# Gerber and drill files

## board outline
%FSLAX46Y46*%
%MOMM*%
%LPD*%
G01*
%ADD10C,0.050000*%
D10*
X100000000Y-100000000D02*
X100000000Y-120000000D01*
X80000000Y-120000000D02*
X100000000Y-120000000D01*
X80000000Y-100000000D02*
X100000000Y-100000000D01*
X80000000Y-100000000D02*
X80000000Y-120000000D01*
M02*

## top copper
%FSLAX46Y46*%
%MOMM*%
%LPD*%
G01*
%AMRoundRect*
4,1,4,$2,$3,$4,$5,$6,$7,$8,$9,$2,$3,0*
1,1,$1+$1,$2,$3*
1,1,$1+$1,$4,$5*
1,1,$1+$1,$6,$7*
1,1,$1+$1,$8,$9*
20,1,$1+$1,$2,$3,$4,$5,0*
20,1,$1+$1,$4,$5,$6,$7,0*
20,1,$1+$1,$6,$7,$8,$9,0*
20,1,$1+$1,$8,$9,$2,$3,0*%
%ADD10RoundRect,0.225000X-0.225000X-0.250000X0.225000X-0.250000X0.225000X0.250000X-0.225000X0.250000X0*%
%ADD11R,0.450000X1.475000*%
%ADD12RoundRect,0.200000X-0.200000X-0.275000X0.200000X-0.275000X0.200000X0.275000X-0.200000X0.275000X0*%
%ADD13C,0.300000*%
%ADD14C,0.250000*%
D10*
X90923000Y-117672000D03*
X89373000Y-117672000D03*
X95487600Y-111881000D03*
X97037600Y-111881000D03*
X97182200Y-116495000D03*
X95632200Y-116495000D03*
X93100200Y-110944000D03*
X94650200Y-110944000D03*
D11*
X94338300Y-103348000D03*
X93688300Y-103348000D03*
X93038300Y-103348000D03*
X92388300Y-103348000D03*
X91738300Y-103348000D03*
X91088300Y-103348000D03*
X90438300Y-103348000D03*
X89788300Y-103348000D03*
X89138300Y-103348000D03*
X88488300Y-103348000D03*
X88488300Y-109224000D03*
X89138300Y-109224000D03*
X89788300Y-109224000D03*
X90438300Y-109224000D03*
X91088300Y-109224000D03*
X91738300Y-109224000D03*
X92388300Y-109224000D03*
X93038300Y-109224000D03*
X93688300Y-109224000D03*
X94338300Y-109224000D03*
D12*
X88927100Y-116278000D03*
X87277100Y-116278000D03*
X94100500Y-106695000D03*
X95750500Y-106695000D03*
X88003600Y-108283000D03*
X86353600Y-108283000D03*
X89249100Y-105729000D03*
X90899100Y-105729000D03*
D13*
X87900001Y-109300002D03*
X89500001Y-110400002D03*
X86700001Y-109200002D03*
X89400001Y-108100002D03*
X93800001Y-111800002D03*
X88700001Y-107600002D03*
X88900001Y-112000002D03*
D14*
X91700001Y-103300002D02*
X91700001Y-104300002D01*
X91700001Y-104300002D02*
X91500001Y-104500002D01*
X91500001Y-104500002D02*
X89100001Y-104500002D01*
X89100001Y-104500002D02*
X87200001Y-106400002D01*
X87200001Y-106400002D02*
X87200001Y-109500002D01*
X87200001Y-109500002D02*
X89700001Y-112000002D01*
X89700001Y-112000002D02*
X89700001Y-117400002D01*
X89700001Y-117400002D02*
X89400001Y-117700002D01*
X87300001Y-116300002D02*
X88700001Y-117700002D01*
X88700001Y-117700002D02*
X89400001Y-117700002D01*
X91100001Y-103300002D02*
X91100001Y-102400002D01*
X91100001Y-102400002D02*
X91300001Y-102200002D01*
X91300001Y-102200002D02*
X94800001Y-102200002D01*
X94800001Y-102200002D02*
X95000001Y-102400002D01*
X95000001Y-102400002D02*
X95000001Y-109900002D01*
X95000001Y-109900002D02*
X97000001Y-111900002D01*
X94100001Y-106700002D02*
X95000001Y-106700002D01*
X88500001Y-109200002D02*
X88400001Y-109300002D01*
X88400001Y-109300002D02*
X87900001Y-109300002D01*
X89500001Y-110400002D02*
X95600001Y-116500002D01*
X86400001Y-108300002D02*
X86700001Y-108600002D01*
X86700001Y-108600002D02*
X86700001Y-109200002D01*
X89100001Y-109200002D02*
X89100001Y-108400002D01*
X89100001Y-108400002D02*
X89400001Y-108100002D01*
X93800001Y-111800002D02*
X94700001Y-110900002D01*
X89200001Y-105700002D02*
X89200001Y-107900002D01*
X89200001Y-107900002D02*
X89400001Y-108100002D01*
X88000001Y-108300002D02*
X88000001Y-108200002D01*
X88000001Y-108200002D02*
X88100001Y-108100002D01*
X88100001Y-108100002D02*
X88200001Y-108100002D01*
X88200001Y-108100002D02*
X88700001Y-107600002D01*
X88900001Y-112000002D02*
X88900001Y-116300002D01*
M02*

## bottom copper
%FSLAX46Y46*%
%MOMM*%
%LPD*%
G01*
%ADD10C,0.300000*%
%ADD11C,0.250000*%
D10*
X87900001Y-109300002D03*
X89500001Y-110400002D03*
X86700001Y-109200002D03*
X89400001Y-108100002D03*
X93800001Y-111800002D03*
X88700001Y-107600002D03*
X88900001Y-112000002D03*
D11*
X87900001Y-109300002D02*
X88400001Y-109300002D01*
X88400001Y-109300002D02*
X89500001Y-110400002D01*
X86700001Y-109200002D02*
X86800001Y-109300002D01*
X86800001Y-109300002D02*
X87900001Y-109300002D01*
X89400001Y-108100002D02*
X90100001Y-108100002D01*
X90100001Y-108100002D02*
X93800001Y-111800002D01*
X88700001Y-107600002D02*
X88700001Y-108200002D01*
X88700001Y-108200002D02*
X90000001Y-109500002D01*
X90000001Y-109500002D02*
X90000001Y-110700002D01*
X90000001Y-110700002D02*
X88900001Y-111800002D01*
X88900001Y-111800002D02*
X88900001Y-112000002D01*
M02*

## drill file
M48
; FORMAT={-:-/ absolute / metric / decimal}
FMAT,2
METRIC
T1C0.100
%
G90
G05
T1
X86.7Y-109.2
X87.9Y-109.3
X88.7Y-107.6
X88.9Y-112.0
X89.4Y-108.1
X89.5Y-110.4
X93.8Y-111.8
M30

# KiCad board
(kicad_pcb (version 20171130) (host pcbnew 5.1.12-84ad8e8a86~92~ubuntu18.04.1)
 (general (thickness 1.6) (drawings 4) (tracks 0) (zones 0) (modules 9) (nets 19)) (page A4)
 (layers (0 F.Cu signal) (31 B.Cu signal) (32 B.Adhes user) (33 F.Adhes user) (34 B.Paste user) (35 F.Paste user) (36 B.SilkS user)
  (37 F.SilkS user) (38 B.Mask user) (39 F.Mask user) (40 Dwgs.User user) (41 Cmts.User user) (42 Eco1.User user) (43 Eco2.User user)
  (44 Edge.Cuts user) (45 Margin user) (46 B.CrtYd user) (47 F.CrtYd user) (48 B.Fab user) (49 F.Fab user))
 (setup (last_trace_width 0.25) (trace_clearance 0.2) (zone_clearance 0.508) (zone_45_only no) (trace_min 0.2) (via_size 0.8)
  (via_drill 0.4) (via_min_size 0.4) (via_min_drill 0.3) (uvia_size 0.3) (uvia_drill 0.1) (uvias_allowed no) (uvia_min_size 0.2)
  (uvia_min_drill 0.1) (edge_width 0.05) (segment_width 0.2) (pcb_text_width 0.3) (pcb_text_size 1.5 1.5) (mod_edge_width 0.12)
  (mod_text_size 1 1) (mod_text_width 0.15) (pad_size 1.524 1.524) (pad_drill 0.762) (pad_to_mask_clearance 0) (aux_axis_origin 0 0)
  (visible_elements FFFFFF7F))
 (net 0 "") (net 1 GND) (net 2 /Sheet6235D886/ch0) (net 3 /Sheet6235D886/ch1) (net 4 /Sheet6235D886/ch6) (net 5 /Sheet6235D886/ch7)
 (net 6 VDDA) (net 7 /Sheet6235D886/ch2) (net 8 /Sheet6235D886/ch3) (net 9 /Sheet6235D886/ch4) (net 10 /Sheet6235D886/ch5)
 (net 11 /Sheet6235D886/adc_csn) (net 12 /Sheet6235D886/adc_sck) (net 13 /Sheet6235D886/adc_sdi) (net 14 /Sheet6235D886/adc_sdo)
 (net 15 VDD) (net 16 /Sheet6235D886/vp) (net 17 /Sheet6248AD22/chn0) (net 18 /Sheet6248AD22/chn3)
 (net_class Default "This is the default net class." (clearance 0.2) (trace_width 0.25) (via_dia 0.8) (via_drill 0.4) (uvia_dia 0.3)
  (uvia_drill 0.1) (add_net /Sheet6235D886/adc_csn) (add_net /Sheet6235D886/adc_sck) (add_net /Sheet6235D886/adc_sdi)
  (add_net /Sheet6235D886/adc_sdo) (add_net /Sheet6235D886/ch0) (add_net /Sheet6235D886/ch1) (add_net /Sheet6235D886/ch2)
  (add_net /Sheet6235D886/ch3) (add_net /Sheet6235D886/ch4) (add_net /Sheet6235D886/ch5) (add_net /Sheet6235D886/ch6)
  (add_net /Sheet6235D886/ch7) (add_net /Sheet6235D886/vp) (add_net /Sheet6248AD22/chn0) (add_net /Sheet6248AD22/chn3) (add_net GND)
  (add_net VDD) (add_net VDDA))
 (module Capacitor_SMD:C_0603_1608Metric (layer F.Cu) (at 90.148000 117.672000)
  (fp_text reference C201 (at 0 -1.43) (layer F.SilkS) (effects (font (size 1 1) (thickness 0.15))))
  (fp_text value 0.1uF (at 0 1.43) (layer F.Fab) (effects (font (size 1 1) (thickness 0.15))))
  (pad 2 smd roundrect (at 0.775 0) (size 0.9 0.95) (layers F.Cu F.Mask F.Paste) (roundrect_rratio 0.25) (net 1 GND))
  (pad 1 smd roundrect (at -0.775 0) (size 0.9 0.95) (layers F.Cu F.Mask F.Paste) (roundrect_rratio 0.25) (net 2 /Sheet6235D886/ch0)))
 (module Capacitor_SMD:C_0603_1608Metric (layer F.Cu) (at 96.262600 111.881000)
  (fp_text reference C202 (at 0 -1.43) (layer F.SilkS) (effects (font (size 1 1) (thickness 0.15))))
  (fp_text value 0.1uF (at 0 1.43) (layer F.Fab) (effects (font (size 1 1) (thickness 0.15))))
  (pad 1 smd roundrect (at -0.775 0) (size 0.9 0.95) (layers F.Cu F.Mask F.Paste) (roundrect_rratio 0.25) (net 1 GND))
  (pad 2 smd roundrect (at 0.775 0) (size 0.9 0.95) (layers F.Cu F.Mask F.Paste) (roundrect_rratio 0.25) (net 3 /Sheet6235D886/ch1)))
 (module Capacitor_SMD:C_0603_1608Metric (layer F.Cu) (at 96.407200 116.495000)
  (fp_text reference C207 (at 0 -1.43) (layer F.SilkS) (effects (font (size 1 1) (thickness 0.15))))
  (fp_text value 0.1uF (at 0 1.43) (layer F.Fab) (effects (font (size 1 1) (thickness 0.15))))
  (pad 2 smd roundrect (at 0.775 0) (size 0.9 0.95) (layers F.Cu F.Mask F.Paste) (roundrect_rratio 0.25) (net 1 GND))
  (pad 1 smd roundrect (at -0.775 0) (size 0.9 0.95) (layers F.Cu F.Mask F.Paste) (roundrect_rratio 0.25) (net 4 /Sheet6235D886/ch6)))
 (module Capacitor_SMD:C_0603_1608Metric (layer F.Cu) (at 93.875200 110.944000)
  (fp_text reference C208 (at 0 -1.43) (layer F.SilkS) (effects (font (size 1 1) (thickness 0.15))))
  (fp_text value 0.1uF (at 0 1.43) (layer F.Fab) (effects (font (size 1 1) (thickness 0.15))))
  (pad 1 smd roundrect (at -0.775 0) (size 0.9 0.95) (layers F.Cu F.Mask F.Paste) (roundrect_rratio 0.25) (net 1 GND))
  (pad 2 smd roundrect (at 0.775 0) (size 0.9 0.95) (layers F.Cu F.Mask F.Paste) (roundrect_rratio 0.25) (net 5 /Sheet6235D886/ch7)))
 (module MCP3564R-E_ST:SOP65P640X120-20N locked (layer F.Cu) (at 91.413300 106.286000 270.000000)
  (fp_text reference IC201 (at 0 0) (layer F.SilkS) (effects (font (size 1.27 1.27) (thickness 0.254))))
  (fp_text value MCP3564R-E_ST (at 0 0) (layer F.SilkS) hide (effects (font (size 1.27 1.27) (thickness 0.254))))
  (pad 1 smd rect (at -2.938 -2.925) (size 0.45 1.475) (layers F.Cu F.Mask F.Paste) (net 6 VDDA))
  (pad 2 smd rect (at -2.938 -2.275) (size 0.45 1.475) (layers F.Cu F.Mask F.Paste) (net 1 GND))
  (pad 3 smd rect (at -2.938 -1.625) (size 0.45 1.475) (layers F.Cu F.Mask F.Paste) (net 1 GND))
  (pad 4 smd rect (at -2.938 -0.975) (size 0.45 1.475) (layers F.Cu F.Mask F.Paste))
  (pad 5 smd rect (at -2.938 -0.325) (size 0.45 1.475) (layers F.Cu F.Mask F.Paste) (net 2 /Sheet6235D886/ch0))
  (pad 6 smd rect (at -2.938 0.325) (size 0.45 1.475) (layers F.Cu F.Mask F.Paste) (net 3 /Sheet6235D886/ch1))
  (pad 7 smd rect (at -2.938 0.975) (size 0.45 1.475) (layers F.Cu F.Mask F.Paste) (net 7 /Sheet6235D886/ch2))
  (pad 8 smd rect (at -2.938 1.625) (size 0.45 1.475) (layers F.Cu F.Mask F.Paste) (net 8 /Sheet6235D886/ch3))
  (pad 9 smd rect (at -2.938 2.275) (size 0.45 1.475) (layers F.Cu F.Mask F.Paste) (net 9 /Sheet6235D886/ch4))
  (pad 10 smd rect (at -2.938 2.925) (size 0.45 1.475) (layers F.Cu F.Mask F.Paste) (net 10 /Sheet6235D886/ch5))
  (pad 11 smd rect (at 2.938 2.925) (size 0.45 1.475) (layers F.Cu F.Mask F.Paste) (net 4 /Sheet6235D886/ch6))
  (pad 12 smd rect (at 2.938 2.275) (size 0.45 1.475) (layers F.Cu F.Mask F.Paste) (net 5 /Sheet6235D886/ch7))
  (pad 13 smd rect (at 2.938 1.625) (size 0.45 1.475) (layers F.Cu F.Mask F.Paste) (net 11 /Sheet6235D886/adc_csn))
  (pad 14 smd rect (at 2.938 0.975) (size 0.45 1.475) (layers F.Cu F.Mask F.Paste) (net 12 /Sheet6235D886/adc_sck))
  (pad 15 smd rect (at 2.938 0.325) (size 0.45 1.475) (layers F.Cu F.Mask F.Paste) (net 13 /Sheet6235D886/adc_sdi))
  (pad 16 smd rect (at 2.938 -0.325) (size 0.45 1.475) (layers F.Cu F.Mask F.Paste) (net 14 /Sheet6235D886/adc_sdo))
  (pad 17 smd rect (at 2.938 -0.975) (size 0.45 1.475) (layers F.Cu F.Mask F.Paste))
  (pad 18 smd rect (at 2.938 -1.625) (size 0.45 1.475) (layers F.Cu F.Mask F.Paste))
  (pad 19 smd rect (at 2.938 -2.275) (size 0.45 1.475) (layers F.Cu F.Mask F.Paste) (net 1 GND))
  (pad 20 smd rect (at 2.938 -2.925) (size 0.45 1.475) (layers F.Cu F.Mask F.Paste) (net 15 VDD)))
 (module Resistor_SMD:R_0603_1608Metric (layer F.Cu) (at 88.102100 116.278000)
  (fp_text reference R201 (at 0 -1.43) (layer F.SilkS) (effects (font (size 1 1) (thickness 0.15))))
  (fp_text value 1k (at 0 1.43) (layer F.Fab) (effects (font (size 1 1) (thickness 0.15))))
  (pad 2 smd roundrect (at 0.825 0) (size 0.8 0.95) (layers F.Cu F.Mask F.Paste) (roundrect_rratio 0.25) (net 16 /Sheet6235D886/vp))
  (pad 1 smd roundrect (at -0.825 0) (size 0.8 0.95) (layers F.Cu F.Mask F.Paste) (roundrect_rratio 0.25) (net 2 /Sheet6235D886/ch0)))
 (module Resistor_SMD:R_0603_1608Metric (layer F.Cu) (at 94.925500 106.695000)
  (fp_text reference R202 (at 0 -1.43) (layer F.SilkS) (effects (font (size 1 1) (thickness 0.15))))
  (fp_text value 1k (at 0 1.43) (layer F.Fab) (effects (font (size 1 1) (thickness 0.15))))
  (pad 1 smd roundrect (at -0.825 0) (size 0.8 0.95) (layers F.Cu F.Mask F.Paste) (roundrect_rratio 0.25) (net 3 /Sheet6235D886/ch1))
  (pad 2 smd roundrect (at 0.825 0) (size 0.8 0.95) (layers F.Cu F.Mask F.Paste) (roundrect_rratio 0.25) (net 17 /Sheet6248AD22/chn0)))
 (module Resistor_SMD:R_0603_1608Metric (layer F.Cu) (at 87.178600 108.283000)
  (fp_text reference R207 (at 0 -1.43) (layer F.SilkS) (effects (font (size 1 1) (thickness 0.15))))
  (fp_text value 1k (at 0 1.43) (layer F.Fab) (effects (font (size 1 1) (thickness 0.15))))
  (pad 2 smd roundrect (at 0.825 0) (size 0.8 0.95) (layers F.Cu F.Mask F.Paste) (roundrect_rratio 0.25) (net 16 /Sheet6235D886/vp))
  (pad 1 smd roundrect (at -0.825 0) (size 0.8 0.95) (layers F.Cu F.Mask F.Paste) (roundrect_rratio 0.25) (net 4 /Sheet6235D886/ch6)))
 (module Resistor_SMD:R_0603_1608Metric (layer F.Cu) (at 90.074100 105.729000)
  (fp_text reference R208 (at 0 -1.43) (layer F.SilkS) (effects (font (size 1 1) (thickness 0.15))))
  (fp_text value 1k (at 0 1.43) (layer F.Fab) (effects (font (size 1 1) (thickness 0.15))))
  (pad 1 smd roundrect (at -0.825 0) (size 0.8 0.95) (layers F.Cu F.Mask F.Paste) (roundrect_rratio 0.25) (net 5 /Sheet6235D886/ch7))
  (pad 2 smd roundrect (at 0.825 0) (size 0.8 0.95) (layers F.Cu F.Mask F.Paste) (roundrect_rratio 0.25) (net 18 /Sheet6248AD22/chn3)))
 (gr_line (start 100 100) (end 100 120) (layer Edge.Cuts) (width 0.05))
 (gr_line (start 80 120) (end 100 120) (layer Edge.Cuts) (width 0.05))
 (gr_line (start 80 100) (end 100 100) (layer Edge.Cuts) (width 0.05))
 (gr_line (start 80 100) (end 80 120) (layer Edge.Cuts) (width 0.05))
 (segment (start 91.700001 103.300002) (end 91.700001 104.300002) (width 0.250000) (layer F.Cu) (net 2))
 (segment (start 91.700001 104.300002) (end 91.500001 104.500002) (width 0.250000) (layer F.Cu) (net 2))
 (segment (start 91.500001 104.500002) (end 89.100001 104.500002) (width 0.250000) (layer F.Cu) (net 2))
 (segment (start 89.100001 104.500002) (end 87.200001 106.400002) (width 0.250000) (layer F.Cu) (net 2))
 (segment (start 87.200001 106.400002) (end 87.200001 109.500002) (width 0.250000) (layer F.Cu) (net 2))
 (segment (start 87.200001 109.500002) (end 89.700001 112.000002) (width 0.250000) (layer F.Cu) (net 2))
 (segment (start 89.700001 112.000002) (end 89.700001 117.400002) (width 0.250000) (layer F.Cu) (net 2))
 (segment (start 89.700001 117.400002) (end 89.400001 117.700002) (width 0.250000) (layer F.Cu) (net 2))
 (segment (start 87.300001 116.300002) (end 88.700001 117.700002) (width 0.250000) (layer F.Cu) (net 2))
 (segment (start 88.700001 117.700002) (end 89.400001 117.700002) (width 0.250000) (layer F.Cu) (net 2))
 (segment (start 91.100001 103.300002) (end 91.100001 102.400002) (width 0.250000) (layer F.Cu) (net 3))
 (segment (start 91.100001 102.400002) (end 91.300001 102.200002) (width 0.250000) (layer F.Cu) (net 3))
 (segment (start 91.300001 102.200002) (end 94.800001 102.200002) (width 0.250000) (layer F.Cu) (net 3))
 (segment (start 94.800001 102.200002) (end 95.000001 102.400002) (width 0.250000) (layer F.Cu) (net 3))
 (segment (start 95.000001 102.400002) (end 95.000001 109.900002) (width 0.250000) (layer F.Cu) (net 3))
 (segment (start 95.000001 109.900002) (end 97.000001 111.900002) (width 0.250000) (layer F.Cu) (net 3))
 (segment (start 94.100001 106.700002) (end 95.000001 106.700002) (width 0.250000) (layer F.Cu) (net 3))
 (segment (start 88.500001 109.200002) (end 88.400001 109.300002) (width 0.250000) (layer F.Cu) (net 4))
 (segment (start 88.400001 109.300002) (end 87.900001 109.300002) (width 0.250000) (layer F.Cu) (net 4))
 (segment (start 87.900001 109.300002) (end 88.400001 109.300002) (width 0.250000) (layer B.Cu) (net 4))
 (segment (start 88.400001 109.300002) (end 89.500001 110.400002) (width 0.250000) (layer B.Cu) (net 4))
 (segment (start 89.500001 110.400002) (end 95.600001 116.500002) (width 0.250000) (layer F.Cu) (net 4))
 (segment (start 86.400001 108.300002) (end 86.700001 108.600002) (width 0.250000) (layer F.Cu) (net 4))
 (segment (start 86.700001 108.600002) (end 86.700001 109.200002) (width 0.250000) (layer F.Cu) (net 4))
 (segment (start 86.700001 109.200002) (end 86.800001 109.300002) (width 0.250000) (layer B.Cu) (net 4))
 (segment (start 86.800001 109.300002) (end 87.900001 109.300002) (width 0.250000) (layer B.Cu) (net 4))
 (via micro (at 87.900001 109.300002) (size 0.300000) (drill 0.100000) (layers F.Cu B.Cu) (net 4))
 (via micro (at 89.500001 110.400002) (size 0.300000) (drill 0.100000) (layers F.Cu B.Cu) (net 4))
 (via micro (at 86.700001 109.200002) (size 0.300000) (drill 0.100000) (layers F.Cu B.Cu) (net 4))
 (segment (start 89.100001 109.200002) (end 89.100001 108.400002) (width 0.250000) (layer F.Cu) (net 5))
 (segment (start 89.100001 108.400002) (end 89.400001 108.100002) (width 0.250000) (layer F.Cu) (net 5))
 (segment (start 89.400001 108.100002) (end 90.100001 108.100002) (width 0.250000) (layer B.Cu) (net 5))
 (segment (start 90.100001 108.100002) (end 93.800001 111.800002) (width 0.250000) (layer B.Cu) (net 5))
 (segment (start 93.800001 111.800002) (end 94.700001 110.900002) (width 0.250000) (layer F.Cu) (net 5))
 (segment (start 89.200001 105.700002) (end 89.200001 107.900002) (width 0.250000) (layer F.Cu) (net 5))
 (segment (start 89.200001 107.900002) (end 89.400001 108.100002) (width 0.250000) (layer F.Cu) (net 5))
 (via micro (at 89.400001 108.100002) (size 0.300000) (drill 0.100000) (layers F.Cu B.Cu) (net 5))
 (via micro (at 93.800001 111.800002) (size 0.300000) (drill 0.100000) (layers F.Cu B.Cu) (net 5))
 (segment (start 88.000001 108.300002) (end 88.000001 108.200002) (width 0.250000) (layer F.Cu) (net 16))
 (segment (start 88.000001 108.200002) (end 88.100001 108.100002) (width 0.250000) (layer F.Cu) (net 16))
 (segment (start 88.100001 108.100002) (end 88.200001 108.100002) (width 0.250000) (layer F.Cu) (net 16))
 (segment (start 88.200001 108.100002) (end 88.700001 107.600002) (width 0.250000) (layer F.Cu) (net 16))
 (segment (start 88.700001 107.600002) (end 88.700001 108.200002) (width 0.250000) (layer B.Cu) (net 16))
 (segment (start 88.700001 108.200002) (end 90.000001 109.500002) (width 0.250000) (layer B.Cu) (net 16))
 (segment (start 90.000001 109.500002) (end 90.000001 110.700002) (width 0.250000) (layer B.Cu) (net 16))
 (segment (start 90.000001 110.700002) (end 88.900001 111.800002) (width 0.250000) (layer B.Cu) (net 16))
 (segment (start 88.900001 111.800002) (end 88.900001 112.000002) (width 0.250000) (layer B.Cu) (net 16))
 (segment (start 88.900001 112.000002) (end 88.900001 116.300002) (width 0.250000) (layer F.Cu) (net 16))
 (via micro (at 88.700001 107.600002) (size 0.300000) (drill 0.100000) (layers F.Cu B.Cu) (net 16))
 (via micro (at 88.900001 112.000002) (size 0.300000) (drill 0.100000) (layers F.Cu B.Cu) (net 16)))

